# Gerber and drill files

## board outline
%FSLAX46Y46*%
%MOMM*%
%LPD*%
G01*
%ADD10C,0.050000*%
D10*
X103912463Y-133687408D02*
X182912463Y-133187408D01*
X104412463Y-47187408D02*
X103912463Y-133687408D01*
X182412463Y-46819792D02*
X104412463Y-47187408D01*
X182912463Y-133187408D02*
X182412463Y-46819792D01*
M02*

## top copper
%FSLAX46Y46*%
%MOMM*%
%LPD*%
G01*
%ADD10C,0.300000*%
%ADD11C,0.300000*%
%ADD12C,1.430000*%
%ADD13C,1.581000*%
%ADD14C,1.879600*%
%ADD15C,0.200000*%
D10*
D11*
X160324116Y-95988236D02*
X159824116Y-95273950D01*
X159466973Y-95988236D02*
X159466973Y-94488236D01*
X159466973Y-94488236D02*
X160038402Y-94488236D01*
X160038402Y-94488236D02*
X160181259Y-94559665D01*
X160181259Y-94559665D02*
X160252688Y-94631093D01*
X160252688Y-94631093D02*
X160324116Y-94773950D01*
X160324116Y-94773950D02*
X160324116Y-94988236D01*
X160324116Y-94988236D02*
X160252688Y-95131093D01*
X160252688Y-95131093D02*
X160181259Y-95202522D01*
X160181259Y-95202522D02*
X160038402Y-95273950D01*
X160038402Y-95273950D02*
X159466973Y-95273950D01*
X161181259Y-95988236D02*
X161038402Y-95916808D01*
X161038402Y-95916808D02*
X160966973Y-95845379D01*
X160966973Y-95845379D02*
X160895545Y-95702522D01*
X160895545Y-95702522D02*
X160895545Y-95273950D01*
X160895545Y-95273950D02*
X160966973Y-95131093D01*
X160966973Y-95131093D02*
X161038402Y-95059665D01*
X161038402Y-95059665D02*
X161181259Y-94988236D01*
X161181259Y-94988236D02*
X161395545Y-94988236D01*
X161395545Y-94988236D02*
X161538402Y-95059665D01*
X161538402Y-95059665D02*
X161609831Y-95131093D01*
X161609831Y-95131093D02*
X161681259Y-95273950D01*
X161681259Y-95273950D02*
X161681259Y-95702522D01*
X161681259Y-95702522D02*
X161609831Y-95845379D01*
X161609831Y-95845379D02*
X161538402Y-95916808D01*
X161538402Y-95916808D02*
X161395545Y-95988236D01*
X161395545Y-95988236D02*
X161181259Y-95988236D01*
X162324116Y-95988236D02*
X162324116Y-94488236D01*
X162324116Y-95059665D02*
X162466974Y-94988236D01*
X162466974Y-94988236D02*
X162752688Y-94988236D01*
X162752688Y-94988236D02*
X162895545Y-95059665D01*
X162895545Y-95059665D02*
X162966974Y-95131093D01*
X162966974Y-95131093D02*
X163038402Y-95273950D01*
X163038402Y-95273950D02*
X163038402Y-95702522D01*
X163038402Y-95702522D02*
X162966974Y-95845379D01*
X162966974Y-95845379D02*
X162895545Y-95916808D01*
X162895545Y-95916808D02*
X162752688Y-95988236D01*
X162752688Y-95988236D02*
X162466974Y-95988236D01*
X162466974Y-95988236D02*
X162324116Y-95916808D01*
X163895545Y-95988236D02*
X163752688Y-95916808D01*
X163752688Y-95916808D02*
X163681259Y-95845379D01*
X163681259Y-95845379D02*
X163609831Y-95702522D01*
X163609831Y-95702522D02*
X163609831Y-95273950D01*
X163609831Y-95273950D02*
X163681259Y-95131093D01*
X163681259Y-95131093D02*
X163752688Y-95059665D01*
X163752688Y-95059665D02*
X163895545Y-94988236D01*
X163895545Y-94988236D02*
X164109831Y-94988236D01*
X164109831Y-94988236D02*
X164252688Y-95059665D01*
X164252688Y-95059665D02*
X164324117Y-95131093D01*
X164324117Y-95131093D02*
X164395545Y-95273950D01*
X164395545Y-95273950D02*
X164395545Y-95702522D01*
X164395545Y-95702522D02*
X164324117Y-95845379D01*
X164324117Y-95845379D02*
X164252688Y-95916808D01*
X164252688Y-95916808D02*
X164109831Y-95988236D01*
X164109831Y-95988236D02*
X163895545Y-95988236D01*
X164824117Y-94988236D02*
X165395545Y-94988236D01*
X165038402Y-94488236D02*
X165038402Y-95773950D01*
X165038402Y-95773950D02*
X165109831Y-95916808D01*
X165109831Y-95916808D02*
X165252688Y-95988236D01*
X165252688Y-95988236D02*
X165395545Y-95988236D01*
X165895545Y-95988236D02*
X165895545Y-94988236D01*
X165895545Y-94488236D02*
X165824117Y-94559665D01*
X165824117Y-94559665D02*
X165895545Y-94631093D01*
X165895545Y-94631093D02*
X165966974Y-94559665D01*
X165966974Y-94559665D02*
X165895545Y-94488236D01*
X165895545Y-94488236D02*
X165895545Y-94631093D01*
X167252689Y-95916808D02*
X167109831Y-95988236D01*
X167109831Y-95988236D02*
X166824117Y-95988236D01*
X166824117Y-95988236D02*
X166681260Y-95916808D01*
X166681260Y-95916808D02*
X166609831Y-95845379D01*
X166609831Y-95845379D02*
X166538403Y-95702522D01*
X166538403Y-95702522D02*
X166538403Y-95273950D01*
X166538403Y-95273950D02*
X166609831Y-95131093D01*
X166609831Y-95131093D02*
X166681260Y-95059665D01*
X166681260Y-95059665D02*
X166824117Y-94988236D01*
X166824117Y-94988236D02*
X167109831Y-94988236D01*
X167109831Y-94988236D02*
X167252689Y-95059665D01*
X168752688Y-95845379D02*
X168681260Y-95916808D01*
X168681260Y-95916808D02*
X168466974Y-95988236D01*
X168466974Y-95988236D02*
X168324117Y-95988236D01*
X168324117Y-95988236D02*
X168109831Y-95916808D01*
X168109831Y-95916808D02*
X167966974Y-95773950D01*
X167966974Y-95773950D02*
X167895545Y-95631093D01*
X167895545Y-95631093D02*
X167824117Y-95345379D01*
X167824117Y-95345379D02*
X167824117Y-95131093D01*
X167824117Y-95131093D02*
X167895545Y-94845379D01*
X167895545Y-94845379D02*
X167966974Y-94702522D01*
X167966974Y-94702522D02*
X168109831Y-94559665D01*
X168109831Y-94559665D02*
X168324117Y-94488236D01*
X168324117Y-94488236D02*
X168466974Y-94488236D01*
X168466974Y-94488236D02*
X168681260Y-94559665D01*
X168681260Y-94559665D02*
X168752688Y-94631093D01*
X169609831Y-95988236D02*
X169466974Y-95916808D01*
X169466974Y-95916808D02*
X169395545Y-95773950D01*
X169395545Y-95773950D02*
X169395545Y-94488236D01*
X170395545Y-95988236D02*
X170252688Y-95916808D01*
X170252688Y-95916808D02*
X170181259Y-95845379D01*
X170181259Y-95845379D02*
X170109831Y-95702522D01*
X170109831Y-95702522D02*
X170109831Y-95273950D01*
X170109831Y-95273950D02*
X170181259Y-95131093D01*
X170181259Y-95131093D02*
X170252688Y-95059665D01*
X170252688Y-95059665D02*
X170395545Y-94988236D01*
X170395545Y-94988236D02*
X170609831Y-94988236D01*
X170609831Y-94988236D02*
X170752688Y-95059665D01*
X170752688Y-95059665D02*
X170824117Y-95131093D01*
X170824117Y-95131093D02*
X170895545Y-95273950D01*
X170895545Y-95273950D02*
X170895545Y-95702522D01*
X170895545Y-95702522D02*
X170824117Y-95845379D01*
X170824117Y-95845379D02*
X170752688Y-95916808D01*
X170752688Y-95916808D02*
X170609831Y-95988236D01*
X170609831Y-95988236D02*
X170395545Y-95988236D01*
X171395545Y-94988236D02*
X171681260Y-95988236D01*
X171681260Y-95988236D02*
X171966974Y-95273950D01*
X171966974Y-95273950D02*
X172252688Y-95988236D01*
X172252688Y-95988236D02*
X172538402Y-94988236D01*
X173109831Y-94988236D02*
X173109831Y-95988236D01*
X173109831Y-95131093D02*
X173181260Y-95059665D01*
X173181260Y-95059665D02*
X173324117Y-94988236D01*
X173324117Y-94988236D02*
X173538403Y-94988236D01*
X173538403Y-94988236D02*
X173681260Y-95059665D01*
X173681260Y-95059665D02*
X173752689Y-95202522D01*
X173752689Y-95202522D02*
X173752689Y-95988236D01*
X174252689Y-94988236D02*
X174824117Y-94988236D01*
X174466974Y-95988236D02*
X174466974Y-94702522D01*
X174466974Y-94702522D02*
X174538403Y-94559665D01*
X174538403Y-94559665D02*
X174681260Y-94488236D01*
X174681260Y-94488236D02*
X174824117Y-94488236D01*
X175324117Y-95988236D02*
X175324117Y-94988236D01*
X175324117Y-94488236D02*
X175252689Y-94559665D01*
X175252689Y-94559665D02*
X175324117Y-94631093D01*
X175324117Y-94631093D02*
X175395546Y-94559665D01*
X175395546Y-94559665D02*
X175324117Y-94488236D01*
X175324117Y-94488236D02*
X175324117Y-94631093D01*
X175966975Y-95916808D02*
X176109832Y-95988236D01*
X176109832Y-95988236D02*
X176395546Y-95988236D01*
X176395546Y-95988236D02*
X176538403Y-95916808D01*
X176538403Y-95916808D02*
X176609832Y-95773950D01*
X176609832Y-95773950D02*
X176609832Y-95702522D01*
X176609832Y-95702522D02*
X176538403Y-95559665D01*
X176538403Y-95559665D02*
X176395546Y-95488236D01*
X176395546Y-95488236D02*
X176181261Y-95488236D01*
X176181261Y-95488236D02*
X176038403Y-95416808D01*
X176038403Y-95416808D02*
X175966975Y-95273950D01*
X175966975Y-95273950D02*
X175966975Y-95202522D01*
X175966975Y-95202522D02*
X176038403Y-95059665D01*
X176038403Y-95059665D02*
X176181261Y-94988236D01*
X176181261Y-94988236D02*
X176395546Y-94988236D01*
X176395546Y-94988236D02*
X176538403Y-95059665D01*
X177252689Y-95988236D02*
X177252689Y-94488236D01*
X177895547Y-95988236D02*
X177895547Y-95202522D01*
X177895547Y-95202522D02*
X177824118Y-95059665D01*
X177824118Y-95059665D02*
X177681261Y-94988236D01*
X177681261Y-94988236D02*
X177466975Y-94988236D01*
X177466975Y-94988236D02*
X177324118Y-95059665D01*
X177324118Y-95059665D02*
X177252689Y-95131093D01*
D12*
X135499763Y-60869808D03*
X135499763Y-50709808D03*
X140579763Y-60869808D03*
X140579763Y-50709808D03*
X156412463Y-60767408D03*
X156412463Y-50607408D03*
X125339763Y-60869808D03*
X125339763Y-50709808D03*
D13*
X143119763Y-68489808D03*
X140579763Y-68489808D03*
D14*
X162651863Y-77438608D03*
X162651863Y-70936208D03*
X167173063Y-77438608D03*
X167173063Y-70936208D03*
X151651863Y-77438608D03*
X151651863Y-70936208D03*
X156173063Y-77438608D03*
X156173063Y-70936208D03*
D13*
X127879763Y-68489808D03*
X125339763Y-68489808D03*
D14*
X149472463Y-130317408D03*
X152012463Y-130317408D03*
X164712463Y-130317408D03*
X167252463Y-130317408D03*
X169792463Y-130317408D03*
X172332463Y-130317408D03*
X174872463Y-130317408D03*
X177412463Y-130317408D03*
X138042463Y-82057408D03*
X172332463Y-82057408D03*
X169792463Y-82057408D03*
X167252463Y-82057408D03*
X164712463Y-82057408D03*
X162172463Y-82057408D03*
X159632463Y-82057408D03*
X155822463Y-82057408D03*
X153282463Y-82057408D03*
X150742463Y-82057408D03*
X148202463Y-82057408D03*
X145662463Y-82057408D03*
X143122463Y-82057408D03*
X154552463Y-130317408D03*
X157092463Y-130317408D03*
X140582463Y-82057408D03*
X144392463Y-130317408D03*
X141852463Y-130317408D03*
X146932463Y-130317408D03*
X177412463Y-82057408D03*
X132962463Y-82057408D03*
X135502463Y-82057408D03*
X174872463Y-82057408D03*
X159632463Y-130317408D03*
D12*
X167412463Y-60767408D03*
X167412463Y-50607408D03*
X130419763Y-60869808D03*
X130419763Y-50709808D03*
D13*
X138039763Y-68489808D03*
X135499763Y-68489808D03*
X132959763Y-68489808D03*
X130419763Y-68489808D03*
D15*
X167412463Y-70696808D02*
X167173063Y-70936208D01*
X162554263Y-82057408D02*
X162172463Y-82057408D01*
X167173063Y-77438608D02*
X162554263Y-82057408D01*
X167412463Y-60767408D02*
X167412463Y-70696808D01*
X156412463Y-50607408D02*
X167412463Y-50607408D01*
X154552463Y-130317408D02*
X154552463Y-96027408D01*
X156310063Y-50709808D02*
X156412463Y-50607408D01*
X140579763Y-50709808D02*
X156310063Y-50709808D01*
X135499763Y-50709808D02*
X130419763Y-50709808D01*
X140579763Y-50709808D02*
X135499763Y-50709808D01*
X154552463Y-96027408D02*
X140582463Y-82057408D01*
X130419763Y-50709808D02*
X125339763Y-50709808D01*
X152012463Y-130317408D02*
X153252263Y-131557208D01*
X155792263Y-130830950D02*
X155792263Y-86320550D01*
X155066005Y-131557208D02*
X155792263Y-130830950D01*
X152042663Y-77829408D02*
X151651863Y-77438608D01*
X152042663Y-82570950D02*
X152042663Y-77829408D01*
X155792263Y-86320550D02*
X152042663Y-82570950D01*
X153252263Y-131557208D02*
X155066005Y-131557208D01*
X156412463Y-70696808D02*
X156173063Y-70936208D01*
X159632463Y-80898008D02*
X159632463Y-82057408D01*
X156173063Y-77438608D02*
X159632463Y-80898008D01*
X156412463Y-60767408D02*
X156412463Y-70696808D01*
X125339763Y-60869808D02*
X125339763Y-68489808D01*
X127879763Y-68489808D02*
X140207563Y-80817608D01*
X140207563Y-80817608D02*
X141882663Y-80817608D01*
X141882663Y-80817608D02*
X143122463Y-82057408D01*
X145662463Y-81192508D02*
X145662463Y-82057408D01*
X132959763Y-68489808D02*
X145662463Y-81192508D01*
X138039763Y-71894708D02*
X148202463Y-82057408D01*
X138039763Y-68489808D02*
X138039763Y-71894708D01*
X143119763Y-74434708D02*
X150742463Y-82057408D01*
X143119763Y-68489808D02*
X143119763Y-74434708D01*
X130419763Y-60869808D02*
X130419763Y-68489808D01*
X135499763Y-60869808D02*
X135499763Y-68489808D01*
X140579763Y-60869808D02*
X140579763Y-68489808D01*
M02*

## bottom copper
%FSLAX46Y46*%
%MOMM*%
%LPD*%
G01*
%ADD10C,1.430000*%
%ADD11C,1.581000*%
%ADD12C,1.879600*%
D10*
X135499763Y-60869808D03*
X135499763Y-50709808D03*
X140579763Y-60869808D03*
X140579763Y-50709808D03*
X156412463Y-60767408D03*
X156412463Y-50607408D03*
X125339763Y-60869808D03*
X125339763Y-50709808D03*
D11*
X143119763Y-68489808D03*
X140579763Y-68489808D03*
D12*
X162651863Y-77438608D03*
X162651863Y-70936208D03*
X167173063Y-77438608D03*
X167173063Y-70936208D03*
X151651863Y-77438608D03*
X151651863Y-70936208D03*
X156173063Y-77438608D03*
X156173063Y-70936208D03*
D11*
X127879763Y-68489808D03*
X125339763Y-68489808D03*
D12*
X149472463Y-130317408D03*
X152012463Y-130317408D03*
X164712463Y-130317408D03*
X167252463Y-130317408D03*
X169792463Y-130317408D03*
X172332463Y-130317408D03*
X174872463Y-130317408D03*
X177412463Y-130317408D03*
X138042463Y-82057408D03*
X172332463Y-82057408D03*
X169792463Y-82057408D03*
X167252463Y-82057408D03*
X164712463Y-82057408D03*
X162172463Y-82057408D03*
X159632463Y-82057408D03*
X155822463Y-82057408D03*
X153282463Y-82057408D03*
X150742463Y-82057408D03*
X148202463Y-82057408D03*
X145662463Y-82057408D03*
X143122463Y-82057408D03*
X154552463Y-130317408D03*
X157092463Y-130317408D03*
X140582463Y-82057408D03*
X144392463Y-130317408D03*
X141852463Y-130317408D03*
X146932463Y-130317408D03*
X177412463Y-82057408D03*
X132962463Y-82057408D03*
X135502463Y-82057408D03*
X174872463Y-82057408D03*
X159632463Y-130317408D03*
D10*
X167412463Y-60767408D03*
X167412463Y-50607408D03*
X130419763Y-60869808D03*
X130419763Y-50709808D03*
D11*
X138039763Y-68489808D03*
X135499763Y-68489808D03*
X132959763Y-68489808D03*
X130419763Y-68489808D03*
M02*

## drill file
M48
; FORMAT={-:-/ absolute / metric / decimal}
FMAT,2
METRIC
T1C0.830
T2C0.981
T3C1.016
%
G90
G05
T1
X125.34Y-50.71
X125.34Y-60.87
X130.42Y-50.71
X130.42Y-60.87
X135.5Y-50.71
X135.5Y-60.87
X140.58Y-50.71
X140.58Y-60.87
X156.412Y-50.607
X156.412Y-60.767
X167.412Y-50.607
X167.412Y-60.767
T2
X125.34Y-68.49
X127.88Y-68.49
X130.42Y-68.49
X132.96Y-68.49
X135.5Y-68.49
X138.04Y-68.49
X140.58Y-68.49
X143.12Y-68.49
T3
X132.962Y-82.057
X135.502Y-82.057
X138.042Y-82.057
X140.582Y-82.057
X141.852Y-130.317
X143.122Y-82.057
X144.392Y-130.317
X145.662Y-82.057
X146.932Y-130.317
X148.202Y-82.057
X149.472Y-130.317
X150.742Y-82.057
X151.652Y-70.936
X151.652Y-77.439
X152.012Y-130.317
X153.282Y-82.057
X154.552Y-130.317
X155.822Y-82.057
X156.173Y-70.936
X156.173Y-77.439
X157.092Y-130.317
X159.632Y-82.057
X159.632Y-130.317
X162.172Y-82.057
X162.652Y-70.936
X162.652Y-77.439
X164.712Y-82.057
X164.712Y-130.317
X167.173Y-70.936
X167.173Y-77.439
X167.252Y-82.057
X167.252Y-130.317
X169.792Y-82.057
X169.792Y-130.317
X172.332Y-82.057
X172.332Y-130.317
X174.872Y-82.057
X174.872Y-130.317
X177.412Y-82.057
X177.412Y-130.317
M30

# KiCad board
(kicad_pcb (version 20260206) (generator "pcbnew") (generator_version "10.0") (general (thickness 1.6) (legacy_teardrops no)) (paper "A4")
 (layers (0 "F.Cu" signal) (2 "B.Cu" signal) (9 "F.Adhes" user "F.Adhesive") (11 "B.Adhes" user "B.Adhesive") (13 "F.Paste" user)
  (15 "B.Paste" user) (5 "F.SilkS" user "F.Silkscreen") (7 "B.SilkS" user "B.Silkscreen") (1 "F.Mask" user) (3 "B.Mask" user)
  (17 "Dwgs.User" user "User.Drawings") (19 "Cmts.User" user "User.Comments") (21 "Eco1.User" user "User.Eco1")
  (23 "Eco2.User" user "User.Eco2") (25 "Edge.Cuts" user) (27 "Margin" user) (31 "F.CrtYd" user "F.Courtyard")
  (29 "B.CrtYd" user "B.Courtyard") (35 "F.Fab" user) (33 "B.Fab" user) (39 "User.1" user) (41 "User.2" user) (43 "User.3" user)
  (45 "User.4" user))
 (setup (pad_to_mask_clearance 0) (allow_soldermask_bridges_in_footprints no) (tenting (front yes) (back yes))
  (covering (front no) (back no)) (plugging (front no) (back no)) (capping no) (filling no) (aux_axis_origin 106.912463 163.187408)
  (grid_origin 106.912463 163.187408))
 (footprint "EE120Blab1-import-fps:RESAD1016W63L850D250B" (layer "F.Cu") (at 135.499763 55.789808 90)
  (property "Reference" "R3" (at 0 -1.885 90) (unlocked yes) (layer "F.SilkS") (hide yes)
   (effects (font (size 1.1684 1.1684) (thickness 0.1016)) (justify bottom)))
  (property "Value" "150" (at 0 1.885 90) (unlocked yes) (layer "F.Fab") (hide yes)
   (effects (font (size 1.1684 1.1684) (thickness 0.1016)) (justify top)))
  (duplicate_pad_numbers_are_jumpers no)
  (pad "1" thru_hole circle (at -5.08 0 90) (size 1.43 1.43) (drill 0.83) (layers "*.Cu" "*.Mask") (remove_unused_layers no) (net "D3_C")
   (solder_mask_margin 0.1016) (thermal_bridge_angle 0))
  (pad "2" thru_hole circle (at 5.08 0 90) (size 1.43 1.43) (drill 0.83) (layers "*.Cu" "*.Mask") (remove_unused_layers no) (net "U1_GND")
   (solder_mask_margin 0.1016) (thermal_bridge_angle 0)))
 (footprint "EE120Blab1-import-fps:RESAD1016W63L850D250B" (layer "F.Cu") (at 140.579763 55.789808 90)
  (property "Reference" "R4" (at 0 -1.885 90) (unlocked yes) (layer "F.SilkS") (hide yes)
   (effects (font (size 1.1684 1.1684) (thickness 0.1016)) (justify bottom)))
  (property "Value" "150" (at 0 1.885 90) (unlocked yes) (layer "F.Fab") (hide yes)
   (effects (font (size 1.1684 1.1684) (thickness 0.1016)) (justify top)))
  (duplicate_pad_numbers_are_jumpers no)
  (pad "1" thru_hole circle (at -5.08 0 90) (size 1.43 1.43) (drill 0.83) (layers "*.Cu" "*.Mask") (remove_unused_layers no) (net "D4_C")
   (solder_mask_margin 0.1016) (thermal_bridge_angle 0))
  (pad "2" thru_hole circle (at 5.08 0 90) (size 1.43 1.43) (drill 0.83) (layers "*.Cu" "*.Mask") (remove_unused_layers no) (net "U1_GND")
   (solder_mask_margin 0.1016) (thermal_bridge_angle 0)))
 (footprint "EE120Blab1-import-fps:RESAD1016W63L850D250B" (layer "F.Cu") (at 156.412463 55.687408 90)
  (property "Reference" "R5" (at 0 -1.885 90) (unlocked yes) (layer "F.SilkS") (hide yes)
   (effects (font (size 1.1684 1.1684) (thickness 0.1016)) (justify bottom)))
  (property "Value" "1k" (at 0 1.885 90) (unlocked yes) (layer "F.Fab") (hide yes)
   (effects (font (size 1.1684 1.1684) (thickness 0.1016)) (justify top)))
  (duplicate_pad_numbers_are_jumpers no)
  (pad "1" thru_hole circle (at -5.08 0 90) (size 1.43 1.43) (drill 0.83) (layers "*.Cu" "*.Mask") (remove_unused_layers no) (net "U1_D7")
   (solder_mask_margin 0.1016) (thermal_bridge_angle 0))
  (pad "2" thru_hole circle (at 5.08 0 90) (size 1.43 1.43) (drill 0.83) (layers "*.Cu" "*.Mask") (remove_unused_layers no) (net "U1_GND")
   (solder_mask_margin 0.1016) (thermal_bridge_angle 0)))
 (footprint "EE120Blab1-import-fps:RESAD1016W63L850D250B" (layer "F.Cu") (at 125.339763 55.789808 90)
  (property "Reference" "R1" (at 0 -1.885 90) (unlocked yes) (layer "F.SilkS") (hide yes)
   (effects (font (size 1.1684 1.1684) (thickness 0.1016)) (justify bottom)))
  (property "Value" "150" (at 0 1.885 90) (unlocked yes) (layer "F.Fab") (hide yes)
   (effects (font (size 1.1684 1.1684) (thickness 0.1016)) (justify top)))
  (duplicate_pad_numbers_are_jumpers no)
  (pad "1" thru_hole circle (at -5.08 0 90) (size 1.43 1.43) (drill 0.83) (layers "*.Cu" "*.Mask") (remove_unused_layers no) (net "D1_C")
   (solder_mask_margin 0.1016) (thermal_bridge_angle 0))
  (pad "2" thru_hole circle (at 5.08 0 90) (size 1.43 1.43) (drill 0.83) (layers "*.Cu" "*.Mask") (remove_unused_layers no) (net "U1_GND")
   (solder_mask_margin 0.1016) (thermal_bridge_angle 0)))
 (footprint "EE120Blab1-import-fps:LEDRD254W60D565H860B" (layer "F.Cu") (at 141.849763 68.489808 180)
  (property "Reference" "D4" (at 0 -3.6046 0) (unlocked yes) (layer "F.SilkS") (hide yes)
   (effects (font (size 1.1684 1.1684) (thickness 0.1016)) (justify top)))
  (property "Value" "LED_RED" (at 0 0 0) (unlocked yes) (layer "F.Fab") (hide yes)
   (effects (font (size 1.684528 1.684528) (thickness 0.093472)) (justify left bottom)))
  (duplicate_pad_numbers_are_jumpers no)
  (pad "1" thru_hole circle (at -1.27 0 180) (size 1.581 1.581) (drill 0.981) (layers "*.Cu" "*.Mask") (remove_unused_layers no)
   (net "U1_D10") (solder_mask_margin 0.1016) (thermal_bridge_angle 0))
  (pad "2" thru_hole circle (at 1.27 0 180) (size 1.581 1.581) (drill 0.981) (layers "*.Cu" "*.Mask") (remove_unused_layers no) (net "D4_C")
   (solder_mask_margin 0.1016) (thermal_bridge_angle 0)))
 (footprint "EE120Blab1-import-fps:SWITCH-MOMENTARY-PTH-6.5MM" (layer "F.Cu") (at 164.912463 74.187408 90)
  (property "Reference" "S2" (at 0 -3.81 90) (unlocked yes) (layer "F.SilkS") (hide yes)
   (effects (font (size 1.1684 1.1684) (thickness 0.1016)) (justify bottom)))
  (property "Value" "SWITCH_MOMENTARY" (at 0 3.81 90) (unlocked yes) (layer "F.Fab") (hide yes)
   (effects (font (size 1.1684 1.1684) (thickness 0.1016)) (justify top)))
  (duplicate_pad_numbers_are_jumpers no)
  (pad "1" thru_hole circle (at -3.2512 -2.2606 90) (size 1.8796 1.8796) (drill 1.016) (layers "*.Cu" "*.Mask") (remove_unused_layers no)
   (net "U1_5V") (solder_mask_margin 0.1016) (thermal_bridge_angle 0))
  (pad "2" thru_hole circle (at 3.2512 -2.2606 90) (size 1.8796 1.8796) (drill 1.016) (layers "*.Cu" "*.Mask") (remove_unused_layers no)
   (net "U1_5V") (solder_mask_margin 0.1016) (thermal_bridge_angle 0))
  (pad "3" thru_hole circle (at -3.2512 2.2606 90) (size 1.8796 1.8796) (drill 1.016) (layers "*.Cu" "*.Mask") (remove_unused_layers no)
   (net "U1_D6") (solder_mask_margin 0.1016) (thermal_bridge_angle 0))
  (pad "4" thru_hole circle (at 3.2512 2.2606 90) (size 1.8796 1.8796) (drill 1.016) (layers "*.Cu" "*.Mask") (remove_unused_layers no)
   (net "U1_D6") (solder_mask_margin 0.1016) (thermal_bridge_angle 0)))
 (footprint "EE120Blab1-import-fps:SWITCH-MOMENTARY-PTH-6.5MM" (layer "F.Cu") (at 153.912463 74.187408 90)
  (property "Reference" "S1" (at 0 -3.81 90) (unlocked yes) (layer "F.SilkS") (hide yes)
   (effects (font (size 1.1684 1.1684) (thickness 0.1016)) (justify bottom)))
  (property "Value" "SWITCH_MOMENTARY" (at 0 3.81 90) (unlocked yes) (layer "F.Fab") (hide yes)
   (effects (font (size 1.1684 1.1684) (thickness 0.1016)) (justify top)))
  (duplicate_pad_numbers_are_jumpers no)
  (pad "1" thru_hole circle (at -3.2512 -2.2606 90) (size 1.8796 1.8796) (drill 1.016) (layers "*.Cu" "*.Mask") (remove_unused_layers no)
   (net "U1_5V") (solder_mask_margin 0.1016) (thermal_bridge_angle 0))
  (pad "2" thru_hole circle (at 3.2512 -2.2606 90) (size 1.8796 1.8796) (drill 1.016) (layers "*.Cu" "*.Mask") (remove_unused_layers no)
   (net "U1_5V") (solder_mask_margin 0.1016) (thermal_bridge_angle 0))
  (pad "3" thru_hole circle (at -3.2512 2.2606 90) (size 1.8796 1.8796) (drill 1.016) (layers "*.Cu" "*.Mask") (remove_unused_layers no)
   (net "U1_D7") (solder_mask_margin 0.1016) (thermal_bridge_angle 0))
  (pad "4" thru_hole circle (at 3.2512 2.2606 90) (size 1.8796 1.8796) (drill 1.016) (layers "*.Cu" "*.Mask") (remove_unused_layers no)
   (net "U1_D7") (solder_mask_margin 0.1016) (thermal_bridge_angle 0)))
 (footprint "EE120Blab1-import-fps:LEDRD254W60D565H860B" (layer "F.Cu") (at 126.609763 68.489808 180)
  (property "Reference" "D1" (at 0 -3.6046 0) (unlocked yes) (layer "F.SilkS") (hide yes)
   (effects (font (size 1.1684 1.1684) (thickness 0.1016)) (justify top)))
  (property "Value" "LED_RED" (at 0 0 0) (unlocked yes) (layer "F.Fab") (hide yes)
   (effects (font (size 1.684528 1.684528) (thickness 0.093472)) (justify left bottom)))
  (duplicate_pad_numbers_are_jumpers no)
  (pad "1" thru_hole circle (at -1.27 0 180) (size 1.581 1.581) (drill 0.981) (layers "*.Cu" "*.Mask") (remove_unused_layers no)
   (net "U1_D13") (solder_mask_margin 0.1016) (thermal_bridge_angle 0))
  (pad "2" thru_hole circle (at 1.27 0 180) (size 1.581 1.581) (drill 0.981) (layers "*.Cu" "*.Mask") (remove_unused_layers no) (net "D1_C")
   (solder_mask_margin 0.1016) (thermal_bridge_angle 0)))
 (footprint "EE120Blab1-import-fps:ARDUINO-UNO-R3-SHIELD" (layer "F.Cu") (at 152.012463 106.187408 -90)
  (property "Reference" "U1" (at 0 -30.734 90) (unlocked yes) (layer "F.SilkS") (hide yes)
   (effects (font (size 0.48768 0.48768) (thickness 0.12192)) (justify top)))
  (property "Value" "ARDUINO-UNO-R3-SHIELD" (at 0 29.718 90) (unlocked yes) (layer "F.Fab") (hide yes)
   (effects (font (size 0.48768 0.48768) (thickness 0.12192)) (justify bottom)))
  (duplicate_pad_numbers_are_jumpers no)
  (pad "3.3V" thru_hole circle (at 24.13 2.54) (size 1.8796 1.8796) (drill 1.016) (layers "*.Cu" "*.Mask") (remove_unused_layers no)
   (solder_mask_margin 0.1016) (thermal_bridge_angle 0))
  (pad "5V" thru_hole circle (at 24.13 0) (size 1.8796 1.8796) (drill 1.016) (layers "*.Cu" "*.Mask") (remove_unused_layers no)
   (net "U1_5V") (solder_mask_margin 0.1016) (thermal_bridge_angle 0))
  (pad "A0" thru_hole circle (at 24.13 -12.7) (size 1.8796 1.8796) (drill 1.016) (layers "*.Cu" "*.Mask") (remove_unused_layers no)
   (solder_mask_margin 0.1016) (thermal_bridge_angle 0))
  (pad "A1" thru_hole circle (at 24.13 -15.24) (size 1.8796 1.8796) (drill 1.016) (layers "*.Cu" "*.Mask") (remove_unused_layers no)
   (solder_mask_margin 0.1016) (thermal_bridge_angle 0))
  (pad "A2" thru_hole circle (at 24.13 -17.78) (size 1.8796 1.8796) (drill 1.016) (layers "*.Cu" "*.Mask") (remove_unused_layers no)
   (solder_mask_margin 0.1016) (thermal_bridge_angle 0))
  (pad "A3" thru_hole circle (at 24.13 -20.32) (size 1.8796 1.8796) (drill 1.016) (layers "*.Cu" "*.Mask") (remove_unused_layers no)
   (solder_mask_margin 0.1016) (thermal_bridge_angle 0))
  (pad "A4" thru_hole circle (at 24.13 -22.86) (size 1.8796 1.8796) (drill 1.016) (layers "*.Cu" "*.Mask") (remove_unused_layers no)
   (solder_mask_margin 0.1016) (thermal_bridge_angle 0))
  (pad "A5" thru_hole circle (at 24.13 -25.4) (size 1.8796 1.8796) (drill 1.016) (layers "*.Cu" "*.Mask") (remove_unused_layers no)
   (solder_mask_margin 0.1016) (thermal_bridge_angle 0))
  (pad "AREF" thru_hole circle (at -24.13 13.97) (size 1.8796 1.8796) (drill 1.016) (layers "*.Cu" "*.Mask") (remove_unused_layers no)
   (solder_mask_margin 0.1016) (thermal_bridge_angle 0))
  (pad "D2" thru_hole circle (at -24.13 -20.32) (size 1.8796 1.8796) (drill 1.016) (layers "*.Cu" "*.Mask") (remove_unused_layers no)
   (solder_mask_margin 0.1016) (thermal_bridge_angle 0))
  (pad "D3" thru_hole circle (at -24.13 -17.78) (size 1.8796 1.8796) (drill 1.016) (layers "*.Cu" "*.Mask") (remove_unused_layers no)
   (solder_mask_margin 0.1016) (thermal_bridge_angle 0))
  (pad "D4" thru_hole circle (at -24.13 -15.24) (size 1.8796 1.8796) (drill 1.016) (layers "*.Cu" "*.Mask") (remove_unused_layers no)
   (solder_mask_margin 0.1016) (thermal_bridge_angle 0))
  (pad "D5" thru_hole circle (at -24.13 -12.7) (size 1.8796 1.8796) (drill 1.016) (layers "*.Cu" "*.Mask") (remove_unused_layers no)
   (solder_mask_margin 0.1016) (thermal_bridge_angle 0))
  (pad "D6" thru_hole circle (at -24.13 -10.16) (size 1.8796 1.8796) (drill 1.016) (layers "*.Cu" "*.Mask") (remove_unused_layers no)
   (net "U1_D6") (solder_mask_margin 0.1016) (thermal_bridge_angle 0))
  (pad "D7" thru_hole circle (at -24.13 -7.62) (size 1.8796 1.8796) (drill 1.016) (layers "*.Cu" "*.Mask") (remove_unused_layers no)
   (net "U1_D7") (solder_mask_margin 0.1016) (thermal_bridge_angle 0))
  (pad "D8" thru_hole circle (at -24.13 -3.81) (size 1.8796 1.8796) (drill 1.016) (layers "*.Cu" "*.Mask") (remove_unused_layers no)
   (solder_mask_margin 0.1016) (thermal_bridge_angle 0))
  (pad "D9" thru_hole circle (at -24.13 -1.27) (size 1.8796 1.8796) (drill 1.016) (layers "*.Cu" "*.Mask") (remove_unused_layers no)
   (solder_mask_margin 0.1016) (thermal_bridge_angle 0))
  (pad "D10" thru_hole circle (at -24.13 1.27) (size 1.8796 1.8796) (drill 1.016) (layers "*.Cu" "*.Mask") (remove_unused_layers no)
   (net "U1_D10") (solder_mask_margin 0.1016) (thermal_bridge_angle 0))
  (pad "D11" thru_hole circle (at -24.13 3.81) (size 1.8796 1.8796) (drill 1.016) (layers "*.Cu" "*.Mask") (remove_unused_layers no)
   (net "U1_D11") (solder_mask_margin 0.1016) (thermal_bridge_angle 0))
  (pad "D12" thru_hole circle (at -24.13 6.35) (size 1.8796 1.8796) (drill 1.016) (layers "*.Cu" "*.Mask") (remove_unused_layers no)
   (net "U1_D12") (solder_mask_margin 0.1016) (thermal_bridge_angle 0))
  (pad "D13" thru_hole circle (at -24.13 8.89) (size 1.8796 1.8796) (drill 1.016) (layers "*.Cu" "*.Mask") (remove_unused_layers no)
   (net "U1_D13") (solder_mask_margin 0.1016) (thermal_bridge_angle 0))
  (pad "GND@0" thru_hole circle (at 24.13 -2.54) (size 1.8796 1.8796) (drill 1.016) (layers "*.Cu" "*.Mask") (remove_unused_layers no)
   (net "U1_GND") (solder_mask_margin 0.1016) (thermal_bridge_angle 0))
  (pad "GND@1" thru_hole circle (at 24.13 -5.08) (size 1.8796 1.8796) (drill 1.016) (layers "*.Cu" "*.Mask") (remove_unused_layers no)
   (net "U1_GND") (solder_mask_margin 0.1016) (thermal_bridge_angle 0))
  (pad "GND@2" thru_hole circle (at -24.13 11.43) (size 1.8796 1.8796) (drill 1.016) (layers "*.Cu" "*.Mask") (remove_unused_layers no)
   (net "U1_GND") (solder_mask_margin 0.1016) (thermal_bridge_angle 0))
  (pad "IOREF" thru_hole circle (at 24.13 7.62) (size 1.8796 1.8796) (drill 1.016) (layers "*.Cu" "*.Mask") (remove_unused_layers no)
   (solder_mask_margin 0.1016) (thermal_bridge_angle 0))
  (pad "NC" thru_hole circle (at 24.13 10.16) (size 1.8796 1.8796) (drill 1.016) (layers "*.Cu" "*.Mask") (remove_unused_layers no)
   (solder_mask_margin 0.1016) (thermal_bridge_angle 0))
  (pad "RES" thru_hole circle (at 24.13 5.08) (size 1.8796 1.8796) (drill 1.016) (layers "*.Cu" "*.Mask") (remove_unused_layers no)
   (solder_mask_margin 0.1016) (thermal_bridge_angle 0))
  (pad "RX" thru_hole circle (at -24.13 -25.4) (size 1.8796 1.8796) (drill 1.016) (layers "*.Cu" "*.Mask") (remove_unused_layers no)
   (solder_mask_margin 0.1016) (thermal_bridge_angle 0))
  (pad "SCL" thru_hole circle (at -24.13 19.05) (size 1.8796 1.8796) (drill 1.016) (layers "*.Cu" "*.Mask") (remove_unused_layers no)
   (solder_mask_margin 0.1016) (thermal_bridge_angle 0))
  (pad "SDA" thru_hole circle (at -24.13 16.51) (size 1.8796 1.8796) (drill 1.016) (layers "*.Cu" "*.Mask") (remove_unused_layers no)
   (solder_mask_margin 0.1016) (thermal_bridge_angle 0))
  (pad "TX" thru_hole circle (at -24.13 -22.86) (size 1.8796 1.8796) (drill 1.016) (layers "*.Cu" "*.Mask") (remove_unused_layers no)
   (solder_mask_margin 0.1016) (thermal_bridge_angle 0))
  (pad "VIN" thru_hole circle (at 24.13 -7.62) (size 1.8796 1.8796) (drill 1.016) (layers "*.Cu" "*.Mask") (remove_unused_layers no)
   (solder_mask_margin 0.1016) (thermal_bridge_angle 0)))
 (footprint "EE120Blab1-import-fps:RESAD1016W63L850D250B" (layer "F.Cu") (at 167.412463 55.687408 90)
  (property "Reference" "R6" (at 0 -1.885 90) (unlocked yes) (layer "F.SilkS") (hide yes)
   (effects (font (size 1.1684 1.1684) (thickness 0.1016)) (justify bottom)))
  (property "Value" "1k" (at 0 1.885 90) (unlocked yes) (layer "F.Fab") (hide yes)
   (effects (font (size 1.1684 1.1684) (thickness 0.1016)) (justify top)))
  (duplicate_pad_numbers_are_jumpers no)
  (pad "1" thru_hole circle (at -5.08 0 90) (size 1.43 1.43) (drill 0.83) (layers "*.Cu" "*.Mask") (remove_unused_layers no) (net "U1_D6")
   (solder_mask_margin 0.1016) (thermal_bridge_angle 0))
  (pad "2" thru_hole circle (at 5.08 0 90) (size 1.43 1.43) (drill 0.83) (layers "*.Cu" "*.Mask") (remove_unused_layers no) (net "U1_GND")
   (solder_mask_margin 0.1016) (thermal_bridge_angle 0)))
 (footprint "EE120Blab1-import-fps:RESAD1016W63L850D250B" (layer "F.Cu") (at 130.419763 55.789808 90)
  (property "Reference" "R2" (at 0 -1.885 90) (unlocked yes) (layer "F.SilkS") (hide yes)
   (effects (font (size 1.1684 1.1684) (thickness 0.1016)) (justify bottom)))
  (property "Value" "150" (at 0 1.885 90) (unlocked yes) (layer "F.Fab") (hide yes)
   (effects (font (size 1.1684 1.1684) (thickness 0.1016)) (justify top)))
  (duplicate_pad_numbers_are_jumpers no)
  (pad "1" thru_hole circle (at -5.08 0 90) (size 1.43 1.43) (drill 0.83) (layers "*.Cu" "*.Mask") (remove_unused_layers no) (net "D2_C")
   (solder_mask_margin 0.1016) (thermal_bridge_angle 0))
  (pad "2" thru_hole circle (at 5.08 0 90) (size 1.43 1.43) (drill 0.83) (layers "*.Cu" "*.Mask") (remove_unused_layers no) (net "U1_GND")
   (solder_mask_margin 0.1016) (thermal_bridge_angle 0)))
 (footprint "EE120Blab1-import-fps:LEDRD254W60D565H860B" (layer "F.Cu") (at 136.769763 68.489808 180)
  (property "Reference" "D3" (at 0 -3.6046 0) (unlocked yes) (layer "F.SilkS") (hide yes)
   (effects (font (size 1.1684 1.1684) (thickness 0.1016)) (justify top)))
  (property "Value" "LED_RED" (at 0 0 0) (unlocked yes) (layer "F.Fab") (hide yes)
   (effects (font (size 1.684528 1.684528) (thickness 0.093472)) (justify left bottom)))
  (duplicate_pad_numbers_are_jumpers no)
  (pad "1" thru_hole circle (at -1.27 0 180) (size 1.581 1.581) (drill 0.981) (layers "*.Cu" "*.Mask") (remove_unused_layers no)
   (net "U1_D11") (solder_mask_margin 0.1016) (thermal_bridge_angle 0))
  (pad "2" thru_hole circle (at 1.27 0 180) (size 1.581 1.581) (drill 0.981) (layers "*.Cu" "*.Mask") (remove_unused_layers no) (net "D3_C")
   (solder_mask_margin 0.1016) (thermal_bridge_angle 0)))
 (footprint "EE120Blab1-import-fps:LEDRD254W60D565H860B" (layer "F.Cu") (at 131.689763 68.489808 180)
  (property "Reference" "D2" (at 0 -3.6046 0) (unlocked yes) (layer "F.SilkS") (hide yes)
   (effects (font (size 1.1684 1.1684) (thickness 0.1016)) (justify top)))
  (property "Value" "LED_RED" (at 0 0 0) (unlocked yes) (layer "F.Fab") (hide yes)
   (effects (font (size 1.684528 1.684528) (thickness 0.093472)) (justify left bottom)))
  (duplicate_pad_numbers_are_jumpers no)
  (pad "1" thru_hole circle (at -1.27 0 180) (size 1.581 1.581) (drill 0.981) (layers "*.Cu" "*.Mask") (remove_unused_layers no)
   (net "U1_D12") (solder_mask_margin 0.1016) (thermal_bridge_angle 0))
  (pad "2" thru_hole circle (at 1.27 0 180) (size 1.581 1.581) (drill 0.981) (layers "*.Cu" "*.Mask") (remove_unused_layers no) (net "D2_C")
   (solder_mask_margin 0.1016) (thermal_bridge_angle 0)))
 (gr_line (start 103.912463 133.687408) (end 182.912463 133.187408) (stroke (width 0.05) (type solid)) (layer "Edge.Cuts"))
 (gr_line (start 104.412463 47.187408) (end 103.912463 133.687408) (stroke (width 0.05) (type solid)) (layer "Edge.Cuts"))
 (gr_line (start 182.412463 46.819792) (end 104.412463 47.187408) (stroke (width 0.05) (type solid)) (layer "Edge.Cuts"))
 (gr_line (start 182.912463 133.187408) (end 182.412463 46.819792) (stroke (width 0.05) (type solid)) (layer "Edge.Cuts"))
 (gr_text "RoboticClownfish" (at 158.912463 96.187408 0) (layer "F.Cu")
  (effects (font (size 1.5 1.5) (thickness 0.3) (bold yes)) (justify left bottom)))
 (segment (start 167.412463 70.696808) (end 167.173063 70.936208) (width 0.2) (layer "F.Cu") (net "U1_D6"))
 (segment (start 162.554263 82.057408) (end 162.172463 82.057408) (width 0.2) (layer "F.Cu") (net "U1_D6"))
 (segment (start 167.173063 77.438608) (end 162.554263 82.057408) (width 0.2) (layer "F.Cu") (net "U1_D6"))
 (segment (start 167.412463 60.767408) (end 167.412463 70.696808) (width 0.2) (layer "F.Cu") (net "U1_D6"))
 (segment (start 156.412463 50.607408) (end 167.412463 50.607408) (width 0.2) (layer "F.Cu") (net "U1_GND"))
 (segment (start 154.552463 130.317408) (end 154.552463 96.027408) (width 0.2) (layer "F.Cu") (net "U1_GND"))
 (segment (start 156.310063 50.709808) (end 156.412463 50.607408) (width 0.2) (layer "F.Cu") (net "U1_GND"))
 (segment (start 140.579763 50.709808) (end 156.310063 50.709808) (width 0.2) (layer "F.Cu") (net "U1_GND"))
 (segment (start 135.499763 50.709808) (end 130.419763 50.709808) (width 0.2) (layer "F.Cu") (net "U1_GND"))
 (segment (start 140.579763 50.709808) (end 135.499763 50.709808) (width 0.2) (layer "F.Cu") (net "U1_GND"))
 (segment (start 154.552463 96.027408) (end 140.582463 82.057408) (width 0.2) (layer "F.Cu") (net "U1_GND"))
 (segment (start 130.419763 50.709808) (end 125.339763 50.709808) (width 0.2) (layer "F.Cu") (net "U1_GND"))
 (segment (start 152.012463 130.317408) (end 153.252263 131.557208) (width 0.2) (layer "F.Cu") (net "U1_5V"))
 (segment (start 155.792263 130.83095) (end 155.792263 86.32055) (width 0.2) (layer "F.Cu") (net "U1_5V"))
 (segment (start 155.066005 131.557208) (end 155.792263 130.83095) (width 0.2) (layer "F.Cu") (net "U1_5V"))
 (segment (start 152.042663 77.829408) (end 151.651863 77.438608) (width 0.2) (layer "F.Cu") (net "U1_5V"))
 (segment (start 152.042663 82.57095) (end 152.042663 77.829408) (width 0.2) (layer "F.Cu") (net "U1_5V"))
 (segment (start 155.792263 86.32055) (end 152.042663 82.57095) (width 0.2) (layer "F.Cu") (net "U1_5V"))
 (segment (start 153.252263 131.557208) (end 155.066005 131.557208) (width 0.2) (layer "F.Cu") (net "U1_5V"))
 (segment (start 156.412463 70.696808) (end 156.173063 70.936208) (width 0.2) (layer "F.Cu") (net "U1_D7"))
 (segment (start 159.632463 80.898008) (end 159.632463 82.057408) (width 0.2) (layer "F.Cu") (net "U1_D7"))
 (segment (start 156.173063 77.438608) (end 159.632463 80.898008) (width 0.2) (layer "F.Cu") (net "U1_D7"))
 (segment (start 156.412463 60.767408) (end 156.412463 70.696808) (width 0.2) (layer "F.Cu") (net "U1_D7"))
 (segment (start 125.339763 60.869808) (end 125.339763 68.489808) (width 0.2) (layer "F.Cu") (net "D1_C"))
 (segment (start 127.879763 68.489808) (end 140.207563 80.817608) (width 0.2) (layer "F.Cu") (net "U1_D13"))
 (segment (start 140.207563 80.817608) (end 141.882663 80.817608) (width 0.2) (layer "F.Cu") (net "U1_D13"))
 (segment (start 141.882663 80.817608) (end 143.122463 82.057408) (width 0.2) (layer "F.Cu") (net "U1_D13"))
 (segment (start 145.662463 81.192508) (end 145.662463 82.057408) (width 0.2) (layer "F.Cu") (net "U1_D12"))
 (segment (start 132.959763 68.489808) (end 145.662463 81.192508) (width 0.2) (layer "F.Cu") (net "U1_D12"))
 (segment (start 138.039763 71.894708) (end 148.202463 82.057408) (width 0.2) (layer "F.Cu") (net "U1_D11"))
 (segment (start 138.039763 68.489808) (end 138.039763 71.894708) (width 0.2) (layer "F.Cu") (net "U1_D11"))
 (segment (start 143.119763 74.434708) (end 150.742463 82.057408) (width 0.2) (layer "F.Cu") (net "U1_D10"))
 (segment (start 143.119763 68.489808) (end 143.119763 74.434708) (width 0.2) (layer "F.Cu") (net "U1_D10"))
 (segment (start 130.419763 60.869808) (end 130.419763 68.489808) (width 0.2) (layer "F.Cu") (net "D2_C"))
 (segment (start 135.499763 60.869808) (end 135.499763 68.489808) (width 0.2) (layer "F.Cu") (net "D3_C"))
 (segment (start 140.579763 60.869808) (end 140.579763 68.489808) (width 0.2) (layer "F.Cu") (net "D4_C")))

